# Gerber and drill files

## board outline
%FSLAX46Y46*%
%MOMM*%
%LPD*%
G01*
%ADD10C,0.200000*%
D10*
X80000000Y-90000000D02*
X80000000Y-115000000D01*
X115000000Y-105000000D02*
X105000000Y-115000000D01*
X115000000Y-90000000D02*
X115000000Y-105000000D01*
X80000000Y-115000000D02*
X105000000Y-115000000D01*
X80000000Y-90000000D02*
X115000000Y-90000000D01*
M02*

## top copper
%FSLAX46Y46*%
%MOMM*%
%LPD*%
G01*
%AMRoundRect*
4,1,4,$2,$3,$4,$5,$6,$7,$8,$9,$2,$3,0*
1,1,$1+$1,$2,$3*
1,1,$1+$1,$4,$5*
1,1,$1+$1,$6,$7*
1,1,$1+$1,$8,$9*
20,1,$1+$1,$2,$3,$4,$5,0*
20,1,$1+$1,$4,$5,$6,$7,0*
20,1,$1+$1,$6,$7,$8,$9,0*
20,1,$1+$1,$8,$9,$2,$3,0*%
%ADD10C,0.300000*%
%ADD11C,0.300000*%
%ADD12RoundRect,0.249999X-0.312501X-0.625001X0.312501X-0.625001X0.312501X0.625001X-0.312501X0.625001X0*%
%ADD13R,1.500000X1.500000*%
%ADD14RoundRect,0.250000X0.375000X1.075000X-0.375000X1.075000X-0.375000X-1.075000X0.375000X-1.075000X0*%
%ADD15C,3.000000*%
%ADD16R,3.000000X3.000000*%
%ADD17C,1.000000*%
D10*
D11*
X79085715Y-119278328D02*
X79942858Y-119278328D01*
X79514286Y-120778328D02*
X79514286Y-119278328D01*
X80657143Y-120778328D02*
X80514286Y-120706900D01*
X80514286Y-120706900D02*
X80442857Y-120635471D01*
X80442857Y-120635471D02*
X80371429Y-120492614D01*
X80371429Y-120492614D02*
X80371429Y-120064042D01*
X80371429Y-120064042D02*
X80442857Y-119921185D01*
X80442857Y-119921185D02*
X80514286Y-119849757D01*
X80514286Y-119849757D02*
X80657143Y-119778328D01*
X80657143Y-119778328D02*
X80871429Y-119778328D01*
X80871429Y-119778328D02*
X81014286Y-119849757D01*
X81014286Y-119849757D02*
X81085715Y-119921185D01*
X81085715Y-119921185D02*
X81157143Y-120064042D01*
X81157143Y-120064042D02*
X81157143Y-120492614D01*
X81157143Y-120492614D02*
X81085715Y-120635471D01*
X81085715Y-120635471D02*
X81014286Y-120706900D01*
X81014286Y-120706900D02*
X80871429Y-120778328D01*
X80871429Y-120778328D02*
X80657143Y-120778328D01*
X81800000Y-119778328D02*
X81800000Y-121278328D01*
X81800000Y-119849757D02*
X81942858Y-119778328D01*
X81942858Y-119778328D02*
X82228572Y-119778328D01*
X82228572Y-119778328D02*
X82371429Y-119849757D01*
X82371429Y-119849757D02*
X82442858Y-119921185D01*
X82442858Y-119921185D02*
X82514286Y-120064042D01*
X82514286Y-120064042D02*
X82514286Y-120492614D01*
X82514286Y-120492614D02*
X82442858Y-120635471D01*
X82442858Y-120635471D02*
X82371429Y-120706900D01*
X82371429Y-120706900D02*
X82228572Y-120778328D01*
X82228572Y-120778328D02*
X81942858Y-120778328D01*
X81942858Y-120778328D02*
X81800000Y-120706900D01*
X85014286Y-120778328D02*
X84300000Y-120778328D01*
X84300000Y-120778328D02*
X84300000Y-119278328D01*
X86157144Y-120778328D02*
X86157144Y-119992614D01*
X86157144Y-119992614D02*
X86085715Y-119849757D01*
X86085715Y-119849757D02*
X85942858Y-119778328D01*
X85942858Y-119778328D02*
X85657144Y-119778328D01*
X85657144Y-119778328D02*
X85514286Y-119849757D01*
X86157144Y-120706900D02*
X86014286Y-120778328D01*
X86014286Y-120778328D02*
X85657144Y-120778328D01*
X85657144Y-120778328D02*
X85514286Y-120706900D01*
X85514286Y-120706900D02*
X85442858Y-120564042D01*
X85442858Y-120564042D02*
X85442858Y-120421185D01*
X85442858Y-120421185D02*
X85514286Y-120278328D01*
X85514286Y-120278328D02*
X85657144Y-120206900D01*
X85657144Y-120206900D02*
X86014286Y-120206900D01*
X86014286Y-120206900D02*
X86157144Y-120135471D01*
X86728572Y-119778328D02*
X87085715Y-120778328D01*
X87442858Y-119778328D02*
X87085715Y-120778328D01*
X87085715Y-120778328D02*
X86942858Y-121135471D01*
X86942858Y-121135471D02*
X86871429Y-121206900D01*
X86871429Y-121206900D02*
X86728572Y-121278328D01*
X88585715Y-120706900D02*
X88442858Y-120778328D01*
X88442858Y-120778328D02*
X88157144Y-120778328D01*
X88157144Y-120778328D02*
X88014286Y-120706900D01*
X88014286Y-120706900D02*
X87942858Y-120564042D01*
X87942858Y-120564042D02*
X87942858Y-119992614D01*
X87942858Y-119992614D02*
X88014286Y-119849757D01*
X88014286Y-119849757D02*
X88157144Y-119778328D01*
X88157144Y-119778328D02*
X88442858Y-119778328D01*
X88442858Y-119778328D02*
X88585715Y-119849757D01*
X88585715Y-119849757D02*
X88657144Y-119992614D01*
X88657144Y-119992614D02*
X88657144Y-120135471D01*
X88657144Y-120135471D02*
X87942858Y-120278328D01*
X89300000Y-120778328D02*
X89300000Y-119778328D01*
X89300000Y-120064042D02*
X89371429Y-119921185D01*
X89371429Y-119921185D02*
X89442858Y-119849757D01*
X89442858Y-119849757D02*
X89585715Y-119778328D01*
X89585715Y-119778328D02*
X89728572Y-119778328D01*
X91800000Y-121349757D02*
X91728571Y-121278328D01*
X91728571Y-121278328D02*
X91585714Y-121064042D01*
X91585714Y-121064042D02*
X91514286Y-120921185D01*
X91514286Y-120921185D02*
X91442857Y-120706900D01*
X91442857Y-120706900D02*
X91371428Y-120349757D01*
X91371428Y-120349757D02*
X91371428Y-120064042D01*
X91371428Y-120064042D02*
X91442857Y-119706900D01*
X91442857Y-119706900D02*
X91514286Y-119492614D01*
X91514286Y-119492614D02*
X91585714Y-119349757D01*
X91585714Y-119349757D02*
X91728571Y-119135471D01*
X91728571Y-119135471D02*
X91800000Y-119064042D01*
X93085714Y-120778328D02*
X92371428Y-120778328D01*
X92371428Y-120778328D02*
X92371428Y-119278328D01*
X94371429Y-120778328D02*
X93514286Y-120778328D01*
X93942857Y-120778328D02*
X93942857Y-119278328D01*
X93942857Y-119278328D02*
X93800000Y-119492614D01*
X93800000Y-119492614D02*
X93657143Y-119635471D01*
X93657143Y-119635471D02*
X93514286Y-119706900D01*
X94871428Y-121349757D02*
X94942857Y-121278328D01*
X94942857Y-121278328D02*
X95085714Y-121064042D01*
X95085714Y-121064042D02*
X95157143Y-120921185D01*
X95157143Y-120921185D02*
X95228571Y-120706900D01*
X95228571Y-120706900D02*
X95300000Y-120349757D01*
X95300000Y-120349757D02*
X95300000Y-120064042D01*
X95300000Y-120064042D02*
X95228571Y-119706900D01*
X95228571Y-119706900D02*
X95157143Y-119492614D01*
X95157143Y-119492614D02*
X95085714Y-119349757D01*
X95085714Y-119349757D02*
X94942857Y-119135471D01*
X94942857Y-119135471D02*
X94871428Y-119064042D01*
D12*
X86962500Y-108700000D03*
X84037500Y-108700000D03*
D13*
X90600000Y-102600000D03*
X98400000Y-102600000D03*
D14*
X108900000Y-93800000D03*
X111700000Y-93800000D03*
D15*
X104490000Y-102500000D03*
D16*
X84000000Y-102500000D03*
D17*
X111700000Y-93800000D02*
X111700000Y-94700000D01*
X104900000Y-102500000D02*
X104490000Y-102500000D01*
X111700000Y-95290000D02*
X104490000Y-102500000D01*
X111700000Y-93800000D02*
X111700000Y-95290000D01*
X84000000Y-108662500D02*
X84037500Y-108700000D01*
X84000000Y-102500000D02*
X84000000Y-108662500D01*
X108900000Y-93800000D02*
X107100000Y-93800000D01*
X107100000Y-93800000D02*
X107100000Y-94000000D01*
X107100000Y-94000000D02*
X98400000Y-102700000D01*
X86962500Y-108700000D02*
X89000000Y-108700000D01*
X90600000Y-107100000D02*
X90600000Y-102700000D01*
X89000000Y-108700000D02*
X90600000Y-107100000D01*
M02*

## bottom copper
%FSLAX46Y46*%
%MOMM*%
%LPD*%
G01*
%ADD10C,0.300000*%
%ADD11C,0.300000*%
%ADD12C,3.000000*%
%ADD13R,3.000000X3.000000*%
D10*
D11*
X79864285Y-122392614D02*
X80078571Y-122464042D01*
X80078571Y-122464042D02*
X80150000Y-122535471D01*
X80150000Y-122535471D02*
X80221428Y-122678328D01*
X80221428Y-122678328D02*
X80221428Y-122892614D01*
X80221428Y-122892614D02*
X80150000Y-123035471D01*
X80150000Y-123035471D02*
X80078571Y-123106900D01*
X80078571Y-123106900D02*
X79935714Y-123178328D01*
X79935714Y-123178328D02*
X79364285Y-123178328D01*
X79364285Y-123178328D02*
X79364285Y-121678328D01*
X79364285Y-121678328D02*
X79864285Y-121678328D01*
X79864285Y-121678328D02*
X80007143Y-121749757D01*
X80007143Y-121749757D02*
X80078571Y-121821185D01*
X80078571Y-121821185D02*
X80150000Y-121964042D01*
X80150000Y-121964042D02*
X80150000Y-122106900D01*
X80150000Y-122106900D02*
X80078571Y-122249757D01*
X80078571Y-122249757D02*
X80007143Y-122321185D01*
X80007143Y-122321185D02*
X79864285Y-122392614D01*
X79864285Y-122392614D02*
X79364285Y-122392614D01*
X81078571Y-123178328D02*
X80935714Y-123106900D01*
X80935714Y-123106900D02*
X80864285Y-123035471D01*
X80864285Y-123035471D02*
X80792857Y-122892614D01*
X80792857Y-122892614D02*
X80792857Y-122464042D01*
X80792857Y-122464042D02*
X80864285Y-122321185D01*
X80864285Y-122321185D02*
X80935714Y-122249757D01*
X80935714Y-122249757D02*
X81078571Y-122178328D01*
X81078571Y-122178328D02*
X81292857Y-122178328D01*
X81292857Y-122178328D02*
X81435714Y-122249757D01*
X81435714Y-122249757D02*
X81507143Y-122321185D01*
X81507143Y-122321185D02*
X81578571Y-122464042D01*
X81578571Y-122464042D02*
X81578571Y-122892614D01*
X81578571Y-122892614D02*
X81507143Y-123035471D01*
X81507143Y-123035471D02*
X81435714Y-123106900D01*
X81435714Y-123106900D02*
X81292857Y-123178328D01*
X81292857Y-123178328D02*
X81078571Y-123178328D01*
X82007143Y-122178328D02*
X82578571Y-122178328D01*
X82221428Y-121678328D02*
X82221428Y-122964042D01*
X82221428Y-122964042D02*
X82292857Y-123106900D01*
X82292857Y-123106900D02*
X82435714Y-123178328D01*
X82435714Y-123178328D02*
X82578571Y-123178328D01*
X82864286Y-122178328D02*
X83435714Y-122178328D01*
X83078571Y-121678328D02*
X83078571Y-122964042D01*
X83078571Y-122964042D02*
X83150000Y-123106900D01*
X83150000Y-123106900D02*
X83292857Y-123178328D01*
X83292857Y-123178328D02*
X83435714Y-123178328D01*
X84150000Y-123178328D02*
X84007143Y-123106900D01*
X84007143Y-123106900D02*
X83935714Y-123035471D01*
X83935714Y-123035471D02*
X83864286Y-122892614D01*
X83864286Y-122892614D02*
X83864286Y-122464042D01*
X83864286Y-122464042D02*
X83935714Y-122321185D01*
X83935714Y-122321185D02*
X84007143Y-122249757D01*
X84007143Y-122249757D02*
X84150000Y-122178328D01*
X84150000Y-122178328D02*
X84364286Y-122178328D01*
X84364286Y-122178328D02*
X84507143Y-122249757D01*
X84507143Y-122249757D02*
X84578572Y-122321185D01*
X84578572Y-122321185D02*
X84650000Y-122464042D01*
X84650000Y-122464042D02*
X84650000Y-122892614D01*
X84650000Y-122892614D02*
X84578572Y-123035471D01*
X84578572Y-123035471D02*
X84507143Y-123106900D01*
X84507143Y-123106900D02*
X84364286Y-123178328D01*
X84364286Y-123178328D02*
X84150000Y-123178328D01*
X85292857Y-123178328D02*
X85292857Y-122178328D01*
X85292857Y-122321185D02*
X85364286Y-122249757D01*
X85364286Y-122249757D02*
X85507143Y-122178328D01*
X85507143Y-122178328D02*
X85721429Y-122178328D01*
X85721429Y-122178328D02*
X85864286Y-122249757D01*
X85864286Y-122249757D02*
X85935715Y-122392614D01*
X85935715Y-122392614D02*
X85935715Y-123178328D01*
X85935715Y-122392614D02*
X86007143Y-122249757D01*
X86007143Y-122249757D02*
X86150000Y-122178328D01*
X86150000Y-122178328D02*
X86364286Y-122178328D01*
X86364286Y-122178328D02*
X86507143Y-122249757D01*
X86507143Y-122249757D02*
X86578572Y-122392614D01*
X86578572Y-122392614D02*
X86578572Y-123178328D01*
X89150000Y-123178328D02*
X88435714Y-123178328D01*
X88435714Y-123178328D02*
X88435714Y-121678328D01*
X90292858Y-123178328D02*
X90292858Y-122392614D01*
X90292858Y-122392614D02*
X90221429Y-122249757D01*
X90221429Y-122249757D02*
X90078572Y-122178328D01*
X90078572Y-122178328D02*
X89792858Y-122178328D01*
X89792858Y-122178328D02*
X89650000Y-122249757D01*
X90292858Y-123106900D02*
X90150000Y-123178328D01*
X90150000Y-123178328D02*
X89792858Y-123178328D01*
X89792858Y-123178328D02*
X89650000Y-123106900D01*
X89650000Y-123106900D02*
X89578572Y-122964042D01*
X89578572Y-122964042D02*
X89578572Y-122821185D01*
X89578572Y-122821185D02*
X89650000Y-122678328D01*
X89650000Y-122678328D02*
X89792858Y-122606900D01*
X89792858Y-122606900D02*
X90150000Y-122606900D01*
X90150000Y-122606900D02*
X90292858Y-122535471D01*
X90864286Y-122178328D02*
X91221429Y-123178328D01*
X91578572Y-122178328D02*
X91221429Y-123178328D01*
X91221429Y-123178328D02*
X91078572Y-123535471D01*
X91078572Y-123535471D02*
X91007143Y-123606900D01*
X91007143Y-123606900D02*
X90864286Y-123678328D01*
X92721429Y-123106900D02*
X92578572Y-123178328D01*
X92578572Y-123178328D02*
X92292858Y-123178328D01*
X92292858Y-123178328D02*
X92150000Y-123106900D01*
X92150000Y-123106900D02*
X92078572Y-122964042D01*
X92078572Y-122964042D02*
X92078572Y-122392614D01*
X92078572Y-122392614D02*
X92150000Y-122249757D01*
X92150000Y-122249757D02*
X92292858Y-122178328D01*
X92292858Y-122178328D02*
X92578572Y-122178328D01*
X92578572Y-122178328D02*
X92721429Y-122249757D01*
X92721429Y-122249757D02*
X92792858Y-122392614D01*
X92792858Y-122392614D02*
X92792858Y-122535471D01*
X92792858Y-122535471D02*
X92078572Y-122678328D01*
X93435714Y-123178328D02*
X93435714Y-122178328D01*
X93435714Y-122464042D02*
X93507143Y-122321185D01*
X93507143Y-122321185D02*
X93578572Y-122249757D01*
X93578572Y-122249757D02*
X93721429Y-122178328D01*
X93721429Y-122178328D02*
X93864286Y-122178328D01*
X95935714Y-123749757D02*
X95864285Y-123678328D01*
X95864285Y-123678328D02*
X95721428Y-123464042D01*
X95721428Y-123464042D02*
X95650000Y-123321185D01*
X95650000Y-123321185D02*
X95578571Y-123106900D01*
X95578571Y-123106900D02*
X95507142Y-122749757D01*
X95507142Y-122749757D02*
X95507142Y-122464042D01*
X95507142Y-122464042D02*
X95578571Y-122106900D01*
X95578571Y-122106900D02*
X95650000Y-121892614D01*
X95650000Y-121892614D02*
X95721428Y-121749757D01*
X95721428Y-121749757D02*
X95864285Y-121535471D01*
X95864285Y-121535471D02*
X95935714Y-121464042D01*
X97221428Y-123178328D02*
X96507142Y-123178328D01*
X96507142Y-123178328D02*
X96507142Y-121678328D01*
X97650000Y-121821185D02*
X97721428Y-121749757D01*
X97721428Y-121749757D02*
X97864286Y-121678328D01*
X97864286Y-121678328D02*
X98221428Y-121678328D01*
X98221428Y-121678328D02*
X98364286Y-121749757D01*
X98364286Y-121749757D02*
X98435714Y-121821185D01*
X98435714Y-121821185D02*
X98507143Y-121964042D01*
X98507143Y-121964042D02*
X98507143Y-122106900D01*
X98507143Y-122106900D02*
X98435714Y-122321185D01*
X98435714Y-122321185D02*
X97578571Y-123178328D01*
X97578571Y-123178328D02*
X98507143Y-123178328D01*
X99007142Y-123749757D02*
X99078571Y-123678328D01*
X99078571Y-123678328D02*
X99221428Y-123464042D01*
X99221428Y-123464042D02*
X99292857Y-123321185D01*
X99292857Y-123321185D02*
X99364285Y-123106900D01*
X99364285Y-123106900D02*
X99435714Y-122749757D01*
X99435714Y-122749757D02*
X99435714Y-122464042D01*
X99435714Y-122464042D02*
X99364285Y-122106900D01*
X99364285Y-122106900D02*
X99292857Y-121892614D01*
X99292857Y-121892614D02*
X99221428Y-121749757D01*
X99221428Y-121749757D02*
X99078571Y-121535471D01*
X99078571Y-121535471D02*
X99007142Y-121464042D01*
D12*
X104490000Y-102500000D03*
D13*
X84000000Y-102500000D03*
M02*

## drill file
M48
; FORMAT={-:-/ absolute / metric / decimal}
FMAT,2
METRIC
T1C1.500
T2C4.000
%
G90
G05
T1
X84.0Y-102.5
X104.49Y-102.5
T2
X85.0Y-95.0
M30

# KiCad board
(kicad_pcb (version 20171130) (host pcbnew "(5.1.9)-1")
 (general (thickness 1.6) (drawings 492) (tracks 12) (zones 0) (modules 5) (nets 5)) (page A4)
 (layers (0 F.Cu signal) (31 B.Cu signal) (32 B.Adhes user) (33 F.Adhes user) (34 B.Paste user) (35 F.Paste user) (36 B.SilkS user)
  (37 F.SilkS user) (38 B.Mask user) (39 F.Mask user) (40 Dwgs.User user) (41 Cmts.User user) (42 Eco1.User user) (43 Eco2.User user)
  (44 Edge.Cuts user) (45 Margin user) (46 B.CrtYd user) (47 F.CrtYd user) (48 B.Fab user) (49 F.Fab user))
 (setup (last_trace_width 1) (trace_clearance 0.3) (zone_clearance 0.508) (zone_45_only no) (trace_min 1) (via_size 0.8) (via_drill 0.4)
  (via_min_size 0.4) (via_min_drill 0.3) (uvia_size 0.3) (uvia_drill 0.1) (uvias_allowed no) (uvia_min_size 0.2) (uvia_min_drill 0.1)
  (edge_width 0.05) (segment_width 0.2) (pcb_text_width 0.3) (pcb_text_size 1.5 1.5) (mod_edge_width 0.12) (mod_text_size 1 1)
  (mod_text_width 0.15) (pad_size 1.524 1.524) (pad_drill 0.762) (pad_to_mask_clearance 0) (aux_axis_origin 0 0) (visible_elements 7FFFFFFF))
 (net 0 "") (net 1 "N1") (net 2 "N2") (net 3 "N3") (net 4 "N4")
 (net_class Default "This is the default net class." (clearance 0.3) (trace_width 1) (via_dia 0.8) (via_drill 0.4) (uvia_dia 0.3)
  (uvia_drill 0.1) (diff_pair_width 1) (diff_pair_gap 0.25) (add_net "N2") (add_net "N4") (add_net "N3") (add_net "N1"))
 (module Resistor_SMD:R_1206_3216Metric (layer F.Cu) (at 85.5 108.7)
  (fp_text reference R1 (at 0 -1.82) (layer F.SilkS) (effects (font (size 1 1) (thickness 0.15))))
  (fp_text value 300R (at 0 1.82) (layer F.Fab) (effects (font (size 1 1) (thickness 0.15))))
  (pad 2 smd roundrect (at 1.4625 0) (size 1.125 1.75) (layers F.Cu F.Paste F.Mask) (roundrect_rratio 0.2222213333333333) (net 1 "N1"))
  (pad 1 smd roundrect (at -1.4625 0) (size 1.125 1.75) (layers F.Cu F.Paste F.Mask) (roundrect_rratio 0.2222213333333333) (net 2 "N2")))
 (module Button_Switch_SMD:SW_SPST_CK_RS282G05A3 (layer F.Cu) (at 94.5 102.6 180)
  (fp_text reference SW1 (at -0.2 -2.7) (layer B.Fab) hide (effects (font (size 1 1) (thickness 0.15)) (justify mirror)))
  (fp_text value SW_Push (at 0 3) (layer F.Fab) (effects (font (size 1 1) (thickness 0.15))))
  (pad 2 smd rect (at 3.9 0 180) (size 1.5 1.5) (layers F.Cu F.Paste F.Mask) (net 1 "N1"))
  (pad 1 smd rect (at -3.9 0 180) (size 1.5 1.5) (layers F.Cu F.Paste F.Mask) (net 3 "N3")))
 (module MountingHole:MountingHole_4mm (layer F.Cu) (at 85 95)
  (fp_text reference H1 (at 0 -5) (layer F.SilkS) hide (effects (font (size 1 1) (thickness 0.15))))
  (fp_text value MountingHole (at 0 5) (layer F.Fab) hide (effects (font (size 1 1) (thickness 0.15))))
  (pad 1 np_thru_hole circle (at 0 0) (size 4 4) (drill 4) (layers *.Cu *.Mask)))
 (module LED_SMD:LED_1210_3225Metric (layer F.Cu) (at 110.3 93.8 180)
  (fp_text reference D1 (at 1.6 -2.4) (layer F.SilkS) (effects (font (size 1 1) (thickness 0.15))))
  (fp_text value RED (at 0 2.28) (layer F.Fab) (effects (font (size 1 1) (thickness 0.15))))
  (pad 2 smd roundrect (at 1.4 0 180) (size 1.25 2.65) (layers F.Cu F.Paste F.Mask) (roundrect_rratio 0.2) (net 3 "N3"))
  (pad 1 smd roundrect (at -1.4 0 180) (size 1.25 2.65) (layers F.Cu F.Paste F.Mask) (roundrect_rratio 0.2) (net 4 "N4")))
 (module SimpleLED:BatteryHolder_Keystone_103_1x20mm (layer B.Cu) (at 84 102.5)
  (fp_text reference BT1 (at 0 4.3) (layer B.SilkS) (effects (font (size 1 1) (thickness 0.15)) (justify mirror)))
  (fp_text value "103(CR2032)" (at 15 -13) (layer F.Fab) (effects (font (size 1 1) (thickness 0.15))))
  (pad 2 thru_hole circle (at 20.49 0) (size 3 3) (drill 1.5) (layers *.Cu *.Mask) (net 4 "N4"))
  (pad 1 thru_hole rect (at 0 0) (size 3 3) (drill 1.5) (layers *.Cu *.Mask) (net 2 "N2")))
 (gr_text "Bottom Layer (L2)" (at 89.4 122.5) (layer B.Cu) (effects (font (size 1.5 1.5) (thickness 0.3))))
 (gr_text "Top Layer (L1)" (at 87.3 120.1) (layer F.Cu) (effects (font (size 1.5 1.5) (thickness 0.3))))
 (gr_line (start 80 90) (end 80 115) (layer Edge.Cuts) (width 0.2))
 (gr_line (start 115 105) (end 105 115) (layer Edge.Cuts) (width 0.2))
 (gr_line (start 115 90) (end 115 105) (layer Edge.Cuts) (width 0.2))
 (gr_line (start 80 115) (end 105 115) (layer Edge.Cuts) (width 0.2))
 (gr_line (start 80 90) (end 115 90) (layer Edge.Cuts) (width 0.2))
 (segment (start 111.7 93.8) (end 111.7 94.7) (width 1) (layer F.Cu) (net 4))
 (segment (start 104.9 102.5) (end 104.49 102.5) (width 1) (layer F.Cu) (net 4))
 (segment (start 111.7 95.29) (end 104.49 102.5) (width 1) (layer F.Cu) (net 4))
 (segment (start 111.7 93.8) (end 111.7 95.29) (width 1) (layer F.Cu) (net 4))
 (segment (start 84 108.6625) (end 84.0375 108.7) (width 1) (layer F.Cu) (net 2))
 (segment (start 84 102.5) (end 84 108.6625) (width 1) (layer F.Cu) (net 2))
 (segment (start 108.9 93.8) (end 107.1 93.8) (width 1) (layer F.Cu) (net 3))
 (segment (start 107.1 93.8) (end 107.1 94) (width 1) (layer F.Cu) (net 3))
 (segment (start 107.1 94) (end 98.4 102.7) (width 1) (layer F.Cu) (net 3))
 (segment (start 86.9625 108.7) (end 89 108.7) (width 1) (layer F.Cu) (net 1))
 (segment (start 90.6 107.1) (end 90.6 102.7) (width 1) (layer F.Cu) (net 1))
 (segment (start 89 108.7) (end 90.6 107.1) (width 1) (layer F.Cu) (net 1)))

